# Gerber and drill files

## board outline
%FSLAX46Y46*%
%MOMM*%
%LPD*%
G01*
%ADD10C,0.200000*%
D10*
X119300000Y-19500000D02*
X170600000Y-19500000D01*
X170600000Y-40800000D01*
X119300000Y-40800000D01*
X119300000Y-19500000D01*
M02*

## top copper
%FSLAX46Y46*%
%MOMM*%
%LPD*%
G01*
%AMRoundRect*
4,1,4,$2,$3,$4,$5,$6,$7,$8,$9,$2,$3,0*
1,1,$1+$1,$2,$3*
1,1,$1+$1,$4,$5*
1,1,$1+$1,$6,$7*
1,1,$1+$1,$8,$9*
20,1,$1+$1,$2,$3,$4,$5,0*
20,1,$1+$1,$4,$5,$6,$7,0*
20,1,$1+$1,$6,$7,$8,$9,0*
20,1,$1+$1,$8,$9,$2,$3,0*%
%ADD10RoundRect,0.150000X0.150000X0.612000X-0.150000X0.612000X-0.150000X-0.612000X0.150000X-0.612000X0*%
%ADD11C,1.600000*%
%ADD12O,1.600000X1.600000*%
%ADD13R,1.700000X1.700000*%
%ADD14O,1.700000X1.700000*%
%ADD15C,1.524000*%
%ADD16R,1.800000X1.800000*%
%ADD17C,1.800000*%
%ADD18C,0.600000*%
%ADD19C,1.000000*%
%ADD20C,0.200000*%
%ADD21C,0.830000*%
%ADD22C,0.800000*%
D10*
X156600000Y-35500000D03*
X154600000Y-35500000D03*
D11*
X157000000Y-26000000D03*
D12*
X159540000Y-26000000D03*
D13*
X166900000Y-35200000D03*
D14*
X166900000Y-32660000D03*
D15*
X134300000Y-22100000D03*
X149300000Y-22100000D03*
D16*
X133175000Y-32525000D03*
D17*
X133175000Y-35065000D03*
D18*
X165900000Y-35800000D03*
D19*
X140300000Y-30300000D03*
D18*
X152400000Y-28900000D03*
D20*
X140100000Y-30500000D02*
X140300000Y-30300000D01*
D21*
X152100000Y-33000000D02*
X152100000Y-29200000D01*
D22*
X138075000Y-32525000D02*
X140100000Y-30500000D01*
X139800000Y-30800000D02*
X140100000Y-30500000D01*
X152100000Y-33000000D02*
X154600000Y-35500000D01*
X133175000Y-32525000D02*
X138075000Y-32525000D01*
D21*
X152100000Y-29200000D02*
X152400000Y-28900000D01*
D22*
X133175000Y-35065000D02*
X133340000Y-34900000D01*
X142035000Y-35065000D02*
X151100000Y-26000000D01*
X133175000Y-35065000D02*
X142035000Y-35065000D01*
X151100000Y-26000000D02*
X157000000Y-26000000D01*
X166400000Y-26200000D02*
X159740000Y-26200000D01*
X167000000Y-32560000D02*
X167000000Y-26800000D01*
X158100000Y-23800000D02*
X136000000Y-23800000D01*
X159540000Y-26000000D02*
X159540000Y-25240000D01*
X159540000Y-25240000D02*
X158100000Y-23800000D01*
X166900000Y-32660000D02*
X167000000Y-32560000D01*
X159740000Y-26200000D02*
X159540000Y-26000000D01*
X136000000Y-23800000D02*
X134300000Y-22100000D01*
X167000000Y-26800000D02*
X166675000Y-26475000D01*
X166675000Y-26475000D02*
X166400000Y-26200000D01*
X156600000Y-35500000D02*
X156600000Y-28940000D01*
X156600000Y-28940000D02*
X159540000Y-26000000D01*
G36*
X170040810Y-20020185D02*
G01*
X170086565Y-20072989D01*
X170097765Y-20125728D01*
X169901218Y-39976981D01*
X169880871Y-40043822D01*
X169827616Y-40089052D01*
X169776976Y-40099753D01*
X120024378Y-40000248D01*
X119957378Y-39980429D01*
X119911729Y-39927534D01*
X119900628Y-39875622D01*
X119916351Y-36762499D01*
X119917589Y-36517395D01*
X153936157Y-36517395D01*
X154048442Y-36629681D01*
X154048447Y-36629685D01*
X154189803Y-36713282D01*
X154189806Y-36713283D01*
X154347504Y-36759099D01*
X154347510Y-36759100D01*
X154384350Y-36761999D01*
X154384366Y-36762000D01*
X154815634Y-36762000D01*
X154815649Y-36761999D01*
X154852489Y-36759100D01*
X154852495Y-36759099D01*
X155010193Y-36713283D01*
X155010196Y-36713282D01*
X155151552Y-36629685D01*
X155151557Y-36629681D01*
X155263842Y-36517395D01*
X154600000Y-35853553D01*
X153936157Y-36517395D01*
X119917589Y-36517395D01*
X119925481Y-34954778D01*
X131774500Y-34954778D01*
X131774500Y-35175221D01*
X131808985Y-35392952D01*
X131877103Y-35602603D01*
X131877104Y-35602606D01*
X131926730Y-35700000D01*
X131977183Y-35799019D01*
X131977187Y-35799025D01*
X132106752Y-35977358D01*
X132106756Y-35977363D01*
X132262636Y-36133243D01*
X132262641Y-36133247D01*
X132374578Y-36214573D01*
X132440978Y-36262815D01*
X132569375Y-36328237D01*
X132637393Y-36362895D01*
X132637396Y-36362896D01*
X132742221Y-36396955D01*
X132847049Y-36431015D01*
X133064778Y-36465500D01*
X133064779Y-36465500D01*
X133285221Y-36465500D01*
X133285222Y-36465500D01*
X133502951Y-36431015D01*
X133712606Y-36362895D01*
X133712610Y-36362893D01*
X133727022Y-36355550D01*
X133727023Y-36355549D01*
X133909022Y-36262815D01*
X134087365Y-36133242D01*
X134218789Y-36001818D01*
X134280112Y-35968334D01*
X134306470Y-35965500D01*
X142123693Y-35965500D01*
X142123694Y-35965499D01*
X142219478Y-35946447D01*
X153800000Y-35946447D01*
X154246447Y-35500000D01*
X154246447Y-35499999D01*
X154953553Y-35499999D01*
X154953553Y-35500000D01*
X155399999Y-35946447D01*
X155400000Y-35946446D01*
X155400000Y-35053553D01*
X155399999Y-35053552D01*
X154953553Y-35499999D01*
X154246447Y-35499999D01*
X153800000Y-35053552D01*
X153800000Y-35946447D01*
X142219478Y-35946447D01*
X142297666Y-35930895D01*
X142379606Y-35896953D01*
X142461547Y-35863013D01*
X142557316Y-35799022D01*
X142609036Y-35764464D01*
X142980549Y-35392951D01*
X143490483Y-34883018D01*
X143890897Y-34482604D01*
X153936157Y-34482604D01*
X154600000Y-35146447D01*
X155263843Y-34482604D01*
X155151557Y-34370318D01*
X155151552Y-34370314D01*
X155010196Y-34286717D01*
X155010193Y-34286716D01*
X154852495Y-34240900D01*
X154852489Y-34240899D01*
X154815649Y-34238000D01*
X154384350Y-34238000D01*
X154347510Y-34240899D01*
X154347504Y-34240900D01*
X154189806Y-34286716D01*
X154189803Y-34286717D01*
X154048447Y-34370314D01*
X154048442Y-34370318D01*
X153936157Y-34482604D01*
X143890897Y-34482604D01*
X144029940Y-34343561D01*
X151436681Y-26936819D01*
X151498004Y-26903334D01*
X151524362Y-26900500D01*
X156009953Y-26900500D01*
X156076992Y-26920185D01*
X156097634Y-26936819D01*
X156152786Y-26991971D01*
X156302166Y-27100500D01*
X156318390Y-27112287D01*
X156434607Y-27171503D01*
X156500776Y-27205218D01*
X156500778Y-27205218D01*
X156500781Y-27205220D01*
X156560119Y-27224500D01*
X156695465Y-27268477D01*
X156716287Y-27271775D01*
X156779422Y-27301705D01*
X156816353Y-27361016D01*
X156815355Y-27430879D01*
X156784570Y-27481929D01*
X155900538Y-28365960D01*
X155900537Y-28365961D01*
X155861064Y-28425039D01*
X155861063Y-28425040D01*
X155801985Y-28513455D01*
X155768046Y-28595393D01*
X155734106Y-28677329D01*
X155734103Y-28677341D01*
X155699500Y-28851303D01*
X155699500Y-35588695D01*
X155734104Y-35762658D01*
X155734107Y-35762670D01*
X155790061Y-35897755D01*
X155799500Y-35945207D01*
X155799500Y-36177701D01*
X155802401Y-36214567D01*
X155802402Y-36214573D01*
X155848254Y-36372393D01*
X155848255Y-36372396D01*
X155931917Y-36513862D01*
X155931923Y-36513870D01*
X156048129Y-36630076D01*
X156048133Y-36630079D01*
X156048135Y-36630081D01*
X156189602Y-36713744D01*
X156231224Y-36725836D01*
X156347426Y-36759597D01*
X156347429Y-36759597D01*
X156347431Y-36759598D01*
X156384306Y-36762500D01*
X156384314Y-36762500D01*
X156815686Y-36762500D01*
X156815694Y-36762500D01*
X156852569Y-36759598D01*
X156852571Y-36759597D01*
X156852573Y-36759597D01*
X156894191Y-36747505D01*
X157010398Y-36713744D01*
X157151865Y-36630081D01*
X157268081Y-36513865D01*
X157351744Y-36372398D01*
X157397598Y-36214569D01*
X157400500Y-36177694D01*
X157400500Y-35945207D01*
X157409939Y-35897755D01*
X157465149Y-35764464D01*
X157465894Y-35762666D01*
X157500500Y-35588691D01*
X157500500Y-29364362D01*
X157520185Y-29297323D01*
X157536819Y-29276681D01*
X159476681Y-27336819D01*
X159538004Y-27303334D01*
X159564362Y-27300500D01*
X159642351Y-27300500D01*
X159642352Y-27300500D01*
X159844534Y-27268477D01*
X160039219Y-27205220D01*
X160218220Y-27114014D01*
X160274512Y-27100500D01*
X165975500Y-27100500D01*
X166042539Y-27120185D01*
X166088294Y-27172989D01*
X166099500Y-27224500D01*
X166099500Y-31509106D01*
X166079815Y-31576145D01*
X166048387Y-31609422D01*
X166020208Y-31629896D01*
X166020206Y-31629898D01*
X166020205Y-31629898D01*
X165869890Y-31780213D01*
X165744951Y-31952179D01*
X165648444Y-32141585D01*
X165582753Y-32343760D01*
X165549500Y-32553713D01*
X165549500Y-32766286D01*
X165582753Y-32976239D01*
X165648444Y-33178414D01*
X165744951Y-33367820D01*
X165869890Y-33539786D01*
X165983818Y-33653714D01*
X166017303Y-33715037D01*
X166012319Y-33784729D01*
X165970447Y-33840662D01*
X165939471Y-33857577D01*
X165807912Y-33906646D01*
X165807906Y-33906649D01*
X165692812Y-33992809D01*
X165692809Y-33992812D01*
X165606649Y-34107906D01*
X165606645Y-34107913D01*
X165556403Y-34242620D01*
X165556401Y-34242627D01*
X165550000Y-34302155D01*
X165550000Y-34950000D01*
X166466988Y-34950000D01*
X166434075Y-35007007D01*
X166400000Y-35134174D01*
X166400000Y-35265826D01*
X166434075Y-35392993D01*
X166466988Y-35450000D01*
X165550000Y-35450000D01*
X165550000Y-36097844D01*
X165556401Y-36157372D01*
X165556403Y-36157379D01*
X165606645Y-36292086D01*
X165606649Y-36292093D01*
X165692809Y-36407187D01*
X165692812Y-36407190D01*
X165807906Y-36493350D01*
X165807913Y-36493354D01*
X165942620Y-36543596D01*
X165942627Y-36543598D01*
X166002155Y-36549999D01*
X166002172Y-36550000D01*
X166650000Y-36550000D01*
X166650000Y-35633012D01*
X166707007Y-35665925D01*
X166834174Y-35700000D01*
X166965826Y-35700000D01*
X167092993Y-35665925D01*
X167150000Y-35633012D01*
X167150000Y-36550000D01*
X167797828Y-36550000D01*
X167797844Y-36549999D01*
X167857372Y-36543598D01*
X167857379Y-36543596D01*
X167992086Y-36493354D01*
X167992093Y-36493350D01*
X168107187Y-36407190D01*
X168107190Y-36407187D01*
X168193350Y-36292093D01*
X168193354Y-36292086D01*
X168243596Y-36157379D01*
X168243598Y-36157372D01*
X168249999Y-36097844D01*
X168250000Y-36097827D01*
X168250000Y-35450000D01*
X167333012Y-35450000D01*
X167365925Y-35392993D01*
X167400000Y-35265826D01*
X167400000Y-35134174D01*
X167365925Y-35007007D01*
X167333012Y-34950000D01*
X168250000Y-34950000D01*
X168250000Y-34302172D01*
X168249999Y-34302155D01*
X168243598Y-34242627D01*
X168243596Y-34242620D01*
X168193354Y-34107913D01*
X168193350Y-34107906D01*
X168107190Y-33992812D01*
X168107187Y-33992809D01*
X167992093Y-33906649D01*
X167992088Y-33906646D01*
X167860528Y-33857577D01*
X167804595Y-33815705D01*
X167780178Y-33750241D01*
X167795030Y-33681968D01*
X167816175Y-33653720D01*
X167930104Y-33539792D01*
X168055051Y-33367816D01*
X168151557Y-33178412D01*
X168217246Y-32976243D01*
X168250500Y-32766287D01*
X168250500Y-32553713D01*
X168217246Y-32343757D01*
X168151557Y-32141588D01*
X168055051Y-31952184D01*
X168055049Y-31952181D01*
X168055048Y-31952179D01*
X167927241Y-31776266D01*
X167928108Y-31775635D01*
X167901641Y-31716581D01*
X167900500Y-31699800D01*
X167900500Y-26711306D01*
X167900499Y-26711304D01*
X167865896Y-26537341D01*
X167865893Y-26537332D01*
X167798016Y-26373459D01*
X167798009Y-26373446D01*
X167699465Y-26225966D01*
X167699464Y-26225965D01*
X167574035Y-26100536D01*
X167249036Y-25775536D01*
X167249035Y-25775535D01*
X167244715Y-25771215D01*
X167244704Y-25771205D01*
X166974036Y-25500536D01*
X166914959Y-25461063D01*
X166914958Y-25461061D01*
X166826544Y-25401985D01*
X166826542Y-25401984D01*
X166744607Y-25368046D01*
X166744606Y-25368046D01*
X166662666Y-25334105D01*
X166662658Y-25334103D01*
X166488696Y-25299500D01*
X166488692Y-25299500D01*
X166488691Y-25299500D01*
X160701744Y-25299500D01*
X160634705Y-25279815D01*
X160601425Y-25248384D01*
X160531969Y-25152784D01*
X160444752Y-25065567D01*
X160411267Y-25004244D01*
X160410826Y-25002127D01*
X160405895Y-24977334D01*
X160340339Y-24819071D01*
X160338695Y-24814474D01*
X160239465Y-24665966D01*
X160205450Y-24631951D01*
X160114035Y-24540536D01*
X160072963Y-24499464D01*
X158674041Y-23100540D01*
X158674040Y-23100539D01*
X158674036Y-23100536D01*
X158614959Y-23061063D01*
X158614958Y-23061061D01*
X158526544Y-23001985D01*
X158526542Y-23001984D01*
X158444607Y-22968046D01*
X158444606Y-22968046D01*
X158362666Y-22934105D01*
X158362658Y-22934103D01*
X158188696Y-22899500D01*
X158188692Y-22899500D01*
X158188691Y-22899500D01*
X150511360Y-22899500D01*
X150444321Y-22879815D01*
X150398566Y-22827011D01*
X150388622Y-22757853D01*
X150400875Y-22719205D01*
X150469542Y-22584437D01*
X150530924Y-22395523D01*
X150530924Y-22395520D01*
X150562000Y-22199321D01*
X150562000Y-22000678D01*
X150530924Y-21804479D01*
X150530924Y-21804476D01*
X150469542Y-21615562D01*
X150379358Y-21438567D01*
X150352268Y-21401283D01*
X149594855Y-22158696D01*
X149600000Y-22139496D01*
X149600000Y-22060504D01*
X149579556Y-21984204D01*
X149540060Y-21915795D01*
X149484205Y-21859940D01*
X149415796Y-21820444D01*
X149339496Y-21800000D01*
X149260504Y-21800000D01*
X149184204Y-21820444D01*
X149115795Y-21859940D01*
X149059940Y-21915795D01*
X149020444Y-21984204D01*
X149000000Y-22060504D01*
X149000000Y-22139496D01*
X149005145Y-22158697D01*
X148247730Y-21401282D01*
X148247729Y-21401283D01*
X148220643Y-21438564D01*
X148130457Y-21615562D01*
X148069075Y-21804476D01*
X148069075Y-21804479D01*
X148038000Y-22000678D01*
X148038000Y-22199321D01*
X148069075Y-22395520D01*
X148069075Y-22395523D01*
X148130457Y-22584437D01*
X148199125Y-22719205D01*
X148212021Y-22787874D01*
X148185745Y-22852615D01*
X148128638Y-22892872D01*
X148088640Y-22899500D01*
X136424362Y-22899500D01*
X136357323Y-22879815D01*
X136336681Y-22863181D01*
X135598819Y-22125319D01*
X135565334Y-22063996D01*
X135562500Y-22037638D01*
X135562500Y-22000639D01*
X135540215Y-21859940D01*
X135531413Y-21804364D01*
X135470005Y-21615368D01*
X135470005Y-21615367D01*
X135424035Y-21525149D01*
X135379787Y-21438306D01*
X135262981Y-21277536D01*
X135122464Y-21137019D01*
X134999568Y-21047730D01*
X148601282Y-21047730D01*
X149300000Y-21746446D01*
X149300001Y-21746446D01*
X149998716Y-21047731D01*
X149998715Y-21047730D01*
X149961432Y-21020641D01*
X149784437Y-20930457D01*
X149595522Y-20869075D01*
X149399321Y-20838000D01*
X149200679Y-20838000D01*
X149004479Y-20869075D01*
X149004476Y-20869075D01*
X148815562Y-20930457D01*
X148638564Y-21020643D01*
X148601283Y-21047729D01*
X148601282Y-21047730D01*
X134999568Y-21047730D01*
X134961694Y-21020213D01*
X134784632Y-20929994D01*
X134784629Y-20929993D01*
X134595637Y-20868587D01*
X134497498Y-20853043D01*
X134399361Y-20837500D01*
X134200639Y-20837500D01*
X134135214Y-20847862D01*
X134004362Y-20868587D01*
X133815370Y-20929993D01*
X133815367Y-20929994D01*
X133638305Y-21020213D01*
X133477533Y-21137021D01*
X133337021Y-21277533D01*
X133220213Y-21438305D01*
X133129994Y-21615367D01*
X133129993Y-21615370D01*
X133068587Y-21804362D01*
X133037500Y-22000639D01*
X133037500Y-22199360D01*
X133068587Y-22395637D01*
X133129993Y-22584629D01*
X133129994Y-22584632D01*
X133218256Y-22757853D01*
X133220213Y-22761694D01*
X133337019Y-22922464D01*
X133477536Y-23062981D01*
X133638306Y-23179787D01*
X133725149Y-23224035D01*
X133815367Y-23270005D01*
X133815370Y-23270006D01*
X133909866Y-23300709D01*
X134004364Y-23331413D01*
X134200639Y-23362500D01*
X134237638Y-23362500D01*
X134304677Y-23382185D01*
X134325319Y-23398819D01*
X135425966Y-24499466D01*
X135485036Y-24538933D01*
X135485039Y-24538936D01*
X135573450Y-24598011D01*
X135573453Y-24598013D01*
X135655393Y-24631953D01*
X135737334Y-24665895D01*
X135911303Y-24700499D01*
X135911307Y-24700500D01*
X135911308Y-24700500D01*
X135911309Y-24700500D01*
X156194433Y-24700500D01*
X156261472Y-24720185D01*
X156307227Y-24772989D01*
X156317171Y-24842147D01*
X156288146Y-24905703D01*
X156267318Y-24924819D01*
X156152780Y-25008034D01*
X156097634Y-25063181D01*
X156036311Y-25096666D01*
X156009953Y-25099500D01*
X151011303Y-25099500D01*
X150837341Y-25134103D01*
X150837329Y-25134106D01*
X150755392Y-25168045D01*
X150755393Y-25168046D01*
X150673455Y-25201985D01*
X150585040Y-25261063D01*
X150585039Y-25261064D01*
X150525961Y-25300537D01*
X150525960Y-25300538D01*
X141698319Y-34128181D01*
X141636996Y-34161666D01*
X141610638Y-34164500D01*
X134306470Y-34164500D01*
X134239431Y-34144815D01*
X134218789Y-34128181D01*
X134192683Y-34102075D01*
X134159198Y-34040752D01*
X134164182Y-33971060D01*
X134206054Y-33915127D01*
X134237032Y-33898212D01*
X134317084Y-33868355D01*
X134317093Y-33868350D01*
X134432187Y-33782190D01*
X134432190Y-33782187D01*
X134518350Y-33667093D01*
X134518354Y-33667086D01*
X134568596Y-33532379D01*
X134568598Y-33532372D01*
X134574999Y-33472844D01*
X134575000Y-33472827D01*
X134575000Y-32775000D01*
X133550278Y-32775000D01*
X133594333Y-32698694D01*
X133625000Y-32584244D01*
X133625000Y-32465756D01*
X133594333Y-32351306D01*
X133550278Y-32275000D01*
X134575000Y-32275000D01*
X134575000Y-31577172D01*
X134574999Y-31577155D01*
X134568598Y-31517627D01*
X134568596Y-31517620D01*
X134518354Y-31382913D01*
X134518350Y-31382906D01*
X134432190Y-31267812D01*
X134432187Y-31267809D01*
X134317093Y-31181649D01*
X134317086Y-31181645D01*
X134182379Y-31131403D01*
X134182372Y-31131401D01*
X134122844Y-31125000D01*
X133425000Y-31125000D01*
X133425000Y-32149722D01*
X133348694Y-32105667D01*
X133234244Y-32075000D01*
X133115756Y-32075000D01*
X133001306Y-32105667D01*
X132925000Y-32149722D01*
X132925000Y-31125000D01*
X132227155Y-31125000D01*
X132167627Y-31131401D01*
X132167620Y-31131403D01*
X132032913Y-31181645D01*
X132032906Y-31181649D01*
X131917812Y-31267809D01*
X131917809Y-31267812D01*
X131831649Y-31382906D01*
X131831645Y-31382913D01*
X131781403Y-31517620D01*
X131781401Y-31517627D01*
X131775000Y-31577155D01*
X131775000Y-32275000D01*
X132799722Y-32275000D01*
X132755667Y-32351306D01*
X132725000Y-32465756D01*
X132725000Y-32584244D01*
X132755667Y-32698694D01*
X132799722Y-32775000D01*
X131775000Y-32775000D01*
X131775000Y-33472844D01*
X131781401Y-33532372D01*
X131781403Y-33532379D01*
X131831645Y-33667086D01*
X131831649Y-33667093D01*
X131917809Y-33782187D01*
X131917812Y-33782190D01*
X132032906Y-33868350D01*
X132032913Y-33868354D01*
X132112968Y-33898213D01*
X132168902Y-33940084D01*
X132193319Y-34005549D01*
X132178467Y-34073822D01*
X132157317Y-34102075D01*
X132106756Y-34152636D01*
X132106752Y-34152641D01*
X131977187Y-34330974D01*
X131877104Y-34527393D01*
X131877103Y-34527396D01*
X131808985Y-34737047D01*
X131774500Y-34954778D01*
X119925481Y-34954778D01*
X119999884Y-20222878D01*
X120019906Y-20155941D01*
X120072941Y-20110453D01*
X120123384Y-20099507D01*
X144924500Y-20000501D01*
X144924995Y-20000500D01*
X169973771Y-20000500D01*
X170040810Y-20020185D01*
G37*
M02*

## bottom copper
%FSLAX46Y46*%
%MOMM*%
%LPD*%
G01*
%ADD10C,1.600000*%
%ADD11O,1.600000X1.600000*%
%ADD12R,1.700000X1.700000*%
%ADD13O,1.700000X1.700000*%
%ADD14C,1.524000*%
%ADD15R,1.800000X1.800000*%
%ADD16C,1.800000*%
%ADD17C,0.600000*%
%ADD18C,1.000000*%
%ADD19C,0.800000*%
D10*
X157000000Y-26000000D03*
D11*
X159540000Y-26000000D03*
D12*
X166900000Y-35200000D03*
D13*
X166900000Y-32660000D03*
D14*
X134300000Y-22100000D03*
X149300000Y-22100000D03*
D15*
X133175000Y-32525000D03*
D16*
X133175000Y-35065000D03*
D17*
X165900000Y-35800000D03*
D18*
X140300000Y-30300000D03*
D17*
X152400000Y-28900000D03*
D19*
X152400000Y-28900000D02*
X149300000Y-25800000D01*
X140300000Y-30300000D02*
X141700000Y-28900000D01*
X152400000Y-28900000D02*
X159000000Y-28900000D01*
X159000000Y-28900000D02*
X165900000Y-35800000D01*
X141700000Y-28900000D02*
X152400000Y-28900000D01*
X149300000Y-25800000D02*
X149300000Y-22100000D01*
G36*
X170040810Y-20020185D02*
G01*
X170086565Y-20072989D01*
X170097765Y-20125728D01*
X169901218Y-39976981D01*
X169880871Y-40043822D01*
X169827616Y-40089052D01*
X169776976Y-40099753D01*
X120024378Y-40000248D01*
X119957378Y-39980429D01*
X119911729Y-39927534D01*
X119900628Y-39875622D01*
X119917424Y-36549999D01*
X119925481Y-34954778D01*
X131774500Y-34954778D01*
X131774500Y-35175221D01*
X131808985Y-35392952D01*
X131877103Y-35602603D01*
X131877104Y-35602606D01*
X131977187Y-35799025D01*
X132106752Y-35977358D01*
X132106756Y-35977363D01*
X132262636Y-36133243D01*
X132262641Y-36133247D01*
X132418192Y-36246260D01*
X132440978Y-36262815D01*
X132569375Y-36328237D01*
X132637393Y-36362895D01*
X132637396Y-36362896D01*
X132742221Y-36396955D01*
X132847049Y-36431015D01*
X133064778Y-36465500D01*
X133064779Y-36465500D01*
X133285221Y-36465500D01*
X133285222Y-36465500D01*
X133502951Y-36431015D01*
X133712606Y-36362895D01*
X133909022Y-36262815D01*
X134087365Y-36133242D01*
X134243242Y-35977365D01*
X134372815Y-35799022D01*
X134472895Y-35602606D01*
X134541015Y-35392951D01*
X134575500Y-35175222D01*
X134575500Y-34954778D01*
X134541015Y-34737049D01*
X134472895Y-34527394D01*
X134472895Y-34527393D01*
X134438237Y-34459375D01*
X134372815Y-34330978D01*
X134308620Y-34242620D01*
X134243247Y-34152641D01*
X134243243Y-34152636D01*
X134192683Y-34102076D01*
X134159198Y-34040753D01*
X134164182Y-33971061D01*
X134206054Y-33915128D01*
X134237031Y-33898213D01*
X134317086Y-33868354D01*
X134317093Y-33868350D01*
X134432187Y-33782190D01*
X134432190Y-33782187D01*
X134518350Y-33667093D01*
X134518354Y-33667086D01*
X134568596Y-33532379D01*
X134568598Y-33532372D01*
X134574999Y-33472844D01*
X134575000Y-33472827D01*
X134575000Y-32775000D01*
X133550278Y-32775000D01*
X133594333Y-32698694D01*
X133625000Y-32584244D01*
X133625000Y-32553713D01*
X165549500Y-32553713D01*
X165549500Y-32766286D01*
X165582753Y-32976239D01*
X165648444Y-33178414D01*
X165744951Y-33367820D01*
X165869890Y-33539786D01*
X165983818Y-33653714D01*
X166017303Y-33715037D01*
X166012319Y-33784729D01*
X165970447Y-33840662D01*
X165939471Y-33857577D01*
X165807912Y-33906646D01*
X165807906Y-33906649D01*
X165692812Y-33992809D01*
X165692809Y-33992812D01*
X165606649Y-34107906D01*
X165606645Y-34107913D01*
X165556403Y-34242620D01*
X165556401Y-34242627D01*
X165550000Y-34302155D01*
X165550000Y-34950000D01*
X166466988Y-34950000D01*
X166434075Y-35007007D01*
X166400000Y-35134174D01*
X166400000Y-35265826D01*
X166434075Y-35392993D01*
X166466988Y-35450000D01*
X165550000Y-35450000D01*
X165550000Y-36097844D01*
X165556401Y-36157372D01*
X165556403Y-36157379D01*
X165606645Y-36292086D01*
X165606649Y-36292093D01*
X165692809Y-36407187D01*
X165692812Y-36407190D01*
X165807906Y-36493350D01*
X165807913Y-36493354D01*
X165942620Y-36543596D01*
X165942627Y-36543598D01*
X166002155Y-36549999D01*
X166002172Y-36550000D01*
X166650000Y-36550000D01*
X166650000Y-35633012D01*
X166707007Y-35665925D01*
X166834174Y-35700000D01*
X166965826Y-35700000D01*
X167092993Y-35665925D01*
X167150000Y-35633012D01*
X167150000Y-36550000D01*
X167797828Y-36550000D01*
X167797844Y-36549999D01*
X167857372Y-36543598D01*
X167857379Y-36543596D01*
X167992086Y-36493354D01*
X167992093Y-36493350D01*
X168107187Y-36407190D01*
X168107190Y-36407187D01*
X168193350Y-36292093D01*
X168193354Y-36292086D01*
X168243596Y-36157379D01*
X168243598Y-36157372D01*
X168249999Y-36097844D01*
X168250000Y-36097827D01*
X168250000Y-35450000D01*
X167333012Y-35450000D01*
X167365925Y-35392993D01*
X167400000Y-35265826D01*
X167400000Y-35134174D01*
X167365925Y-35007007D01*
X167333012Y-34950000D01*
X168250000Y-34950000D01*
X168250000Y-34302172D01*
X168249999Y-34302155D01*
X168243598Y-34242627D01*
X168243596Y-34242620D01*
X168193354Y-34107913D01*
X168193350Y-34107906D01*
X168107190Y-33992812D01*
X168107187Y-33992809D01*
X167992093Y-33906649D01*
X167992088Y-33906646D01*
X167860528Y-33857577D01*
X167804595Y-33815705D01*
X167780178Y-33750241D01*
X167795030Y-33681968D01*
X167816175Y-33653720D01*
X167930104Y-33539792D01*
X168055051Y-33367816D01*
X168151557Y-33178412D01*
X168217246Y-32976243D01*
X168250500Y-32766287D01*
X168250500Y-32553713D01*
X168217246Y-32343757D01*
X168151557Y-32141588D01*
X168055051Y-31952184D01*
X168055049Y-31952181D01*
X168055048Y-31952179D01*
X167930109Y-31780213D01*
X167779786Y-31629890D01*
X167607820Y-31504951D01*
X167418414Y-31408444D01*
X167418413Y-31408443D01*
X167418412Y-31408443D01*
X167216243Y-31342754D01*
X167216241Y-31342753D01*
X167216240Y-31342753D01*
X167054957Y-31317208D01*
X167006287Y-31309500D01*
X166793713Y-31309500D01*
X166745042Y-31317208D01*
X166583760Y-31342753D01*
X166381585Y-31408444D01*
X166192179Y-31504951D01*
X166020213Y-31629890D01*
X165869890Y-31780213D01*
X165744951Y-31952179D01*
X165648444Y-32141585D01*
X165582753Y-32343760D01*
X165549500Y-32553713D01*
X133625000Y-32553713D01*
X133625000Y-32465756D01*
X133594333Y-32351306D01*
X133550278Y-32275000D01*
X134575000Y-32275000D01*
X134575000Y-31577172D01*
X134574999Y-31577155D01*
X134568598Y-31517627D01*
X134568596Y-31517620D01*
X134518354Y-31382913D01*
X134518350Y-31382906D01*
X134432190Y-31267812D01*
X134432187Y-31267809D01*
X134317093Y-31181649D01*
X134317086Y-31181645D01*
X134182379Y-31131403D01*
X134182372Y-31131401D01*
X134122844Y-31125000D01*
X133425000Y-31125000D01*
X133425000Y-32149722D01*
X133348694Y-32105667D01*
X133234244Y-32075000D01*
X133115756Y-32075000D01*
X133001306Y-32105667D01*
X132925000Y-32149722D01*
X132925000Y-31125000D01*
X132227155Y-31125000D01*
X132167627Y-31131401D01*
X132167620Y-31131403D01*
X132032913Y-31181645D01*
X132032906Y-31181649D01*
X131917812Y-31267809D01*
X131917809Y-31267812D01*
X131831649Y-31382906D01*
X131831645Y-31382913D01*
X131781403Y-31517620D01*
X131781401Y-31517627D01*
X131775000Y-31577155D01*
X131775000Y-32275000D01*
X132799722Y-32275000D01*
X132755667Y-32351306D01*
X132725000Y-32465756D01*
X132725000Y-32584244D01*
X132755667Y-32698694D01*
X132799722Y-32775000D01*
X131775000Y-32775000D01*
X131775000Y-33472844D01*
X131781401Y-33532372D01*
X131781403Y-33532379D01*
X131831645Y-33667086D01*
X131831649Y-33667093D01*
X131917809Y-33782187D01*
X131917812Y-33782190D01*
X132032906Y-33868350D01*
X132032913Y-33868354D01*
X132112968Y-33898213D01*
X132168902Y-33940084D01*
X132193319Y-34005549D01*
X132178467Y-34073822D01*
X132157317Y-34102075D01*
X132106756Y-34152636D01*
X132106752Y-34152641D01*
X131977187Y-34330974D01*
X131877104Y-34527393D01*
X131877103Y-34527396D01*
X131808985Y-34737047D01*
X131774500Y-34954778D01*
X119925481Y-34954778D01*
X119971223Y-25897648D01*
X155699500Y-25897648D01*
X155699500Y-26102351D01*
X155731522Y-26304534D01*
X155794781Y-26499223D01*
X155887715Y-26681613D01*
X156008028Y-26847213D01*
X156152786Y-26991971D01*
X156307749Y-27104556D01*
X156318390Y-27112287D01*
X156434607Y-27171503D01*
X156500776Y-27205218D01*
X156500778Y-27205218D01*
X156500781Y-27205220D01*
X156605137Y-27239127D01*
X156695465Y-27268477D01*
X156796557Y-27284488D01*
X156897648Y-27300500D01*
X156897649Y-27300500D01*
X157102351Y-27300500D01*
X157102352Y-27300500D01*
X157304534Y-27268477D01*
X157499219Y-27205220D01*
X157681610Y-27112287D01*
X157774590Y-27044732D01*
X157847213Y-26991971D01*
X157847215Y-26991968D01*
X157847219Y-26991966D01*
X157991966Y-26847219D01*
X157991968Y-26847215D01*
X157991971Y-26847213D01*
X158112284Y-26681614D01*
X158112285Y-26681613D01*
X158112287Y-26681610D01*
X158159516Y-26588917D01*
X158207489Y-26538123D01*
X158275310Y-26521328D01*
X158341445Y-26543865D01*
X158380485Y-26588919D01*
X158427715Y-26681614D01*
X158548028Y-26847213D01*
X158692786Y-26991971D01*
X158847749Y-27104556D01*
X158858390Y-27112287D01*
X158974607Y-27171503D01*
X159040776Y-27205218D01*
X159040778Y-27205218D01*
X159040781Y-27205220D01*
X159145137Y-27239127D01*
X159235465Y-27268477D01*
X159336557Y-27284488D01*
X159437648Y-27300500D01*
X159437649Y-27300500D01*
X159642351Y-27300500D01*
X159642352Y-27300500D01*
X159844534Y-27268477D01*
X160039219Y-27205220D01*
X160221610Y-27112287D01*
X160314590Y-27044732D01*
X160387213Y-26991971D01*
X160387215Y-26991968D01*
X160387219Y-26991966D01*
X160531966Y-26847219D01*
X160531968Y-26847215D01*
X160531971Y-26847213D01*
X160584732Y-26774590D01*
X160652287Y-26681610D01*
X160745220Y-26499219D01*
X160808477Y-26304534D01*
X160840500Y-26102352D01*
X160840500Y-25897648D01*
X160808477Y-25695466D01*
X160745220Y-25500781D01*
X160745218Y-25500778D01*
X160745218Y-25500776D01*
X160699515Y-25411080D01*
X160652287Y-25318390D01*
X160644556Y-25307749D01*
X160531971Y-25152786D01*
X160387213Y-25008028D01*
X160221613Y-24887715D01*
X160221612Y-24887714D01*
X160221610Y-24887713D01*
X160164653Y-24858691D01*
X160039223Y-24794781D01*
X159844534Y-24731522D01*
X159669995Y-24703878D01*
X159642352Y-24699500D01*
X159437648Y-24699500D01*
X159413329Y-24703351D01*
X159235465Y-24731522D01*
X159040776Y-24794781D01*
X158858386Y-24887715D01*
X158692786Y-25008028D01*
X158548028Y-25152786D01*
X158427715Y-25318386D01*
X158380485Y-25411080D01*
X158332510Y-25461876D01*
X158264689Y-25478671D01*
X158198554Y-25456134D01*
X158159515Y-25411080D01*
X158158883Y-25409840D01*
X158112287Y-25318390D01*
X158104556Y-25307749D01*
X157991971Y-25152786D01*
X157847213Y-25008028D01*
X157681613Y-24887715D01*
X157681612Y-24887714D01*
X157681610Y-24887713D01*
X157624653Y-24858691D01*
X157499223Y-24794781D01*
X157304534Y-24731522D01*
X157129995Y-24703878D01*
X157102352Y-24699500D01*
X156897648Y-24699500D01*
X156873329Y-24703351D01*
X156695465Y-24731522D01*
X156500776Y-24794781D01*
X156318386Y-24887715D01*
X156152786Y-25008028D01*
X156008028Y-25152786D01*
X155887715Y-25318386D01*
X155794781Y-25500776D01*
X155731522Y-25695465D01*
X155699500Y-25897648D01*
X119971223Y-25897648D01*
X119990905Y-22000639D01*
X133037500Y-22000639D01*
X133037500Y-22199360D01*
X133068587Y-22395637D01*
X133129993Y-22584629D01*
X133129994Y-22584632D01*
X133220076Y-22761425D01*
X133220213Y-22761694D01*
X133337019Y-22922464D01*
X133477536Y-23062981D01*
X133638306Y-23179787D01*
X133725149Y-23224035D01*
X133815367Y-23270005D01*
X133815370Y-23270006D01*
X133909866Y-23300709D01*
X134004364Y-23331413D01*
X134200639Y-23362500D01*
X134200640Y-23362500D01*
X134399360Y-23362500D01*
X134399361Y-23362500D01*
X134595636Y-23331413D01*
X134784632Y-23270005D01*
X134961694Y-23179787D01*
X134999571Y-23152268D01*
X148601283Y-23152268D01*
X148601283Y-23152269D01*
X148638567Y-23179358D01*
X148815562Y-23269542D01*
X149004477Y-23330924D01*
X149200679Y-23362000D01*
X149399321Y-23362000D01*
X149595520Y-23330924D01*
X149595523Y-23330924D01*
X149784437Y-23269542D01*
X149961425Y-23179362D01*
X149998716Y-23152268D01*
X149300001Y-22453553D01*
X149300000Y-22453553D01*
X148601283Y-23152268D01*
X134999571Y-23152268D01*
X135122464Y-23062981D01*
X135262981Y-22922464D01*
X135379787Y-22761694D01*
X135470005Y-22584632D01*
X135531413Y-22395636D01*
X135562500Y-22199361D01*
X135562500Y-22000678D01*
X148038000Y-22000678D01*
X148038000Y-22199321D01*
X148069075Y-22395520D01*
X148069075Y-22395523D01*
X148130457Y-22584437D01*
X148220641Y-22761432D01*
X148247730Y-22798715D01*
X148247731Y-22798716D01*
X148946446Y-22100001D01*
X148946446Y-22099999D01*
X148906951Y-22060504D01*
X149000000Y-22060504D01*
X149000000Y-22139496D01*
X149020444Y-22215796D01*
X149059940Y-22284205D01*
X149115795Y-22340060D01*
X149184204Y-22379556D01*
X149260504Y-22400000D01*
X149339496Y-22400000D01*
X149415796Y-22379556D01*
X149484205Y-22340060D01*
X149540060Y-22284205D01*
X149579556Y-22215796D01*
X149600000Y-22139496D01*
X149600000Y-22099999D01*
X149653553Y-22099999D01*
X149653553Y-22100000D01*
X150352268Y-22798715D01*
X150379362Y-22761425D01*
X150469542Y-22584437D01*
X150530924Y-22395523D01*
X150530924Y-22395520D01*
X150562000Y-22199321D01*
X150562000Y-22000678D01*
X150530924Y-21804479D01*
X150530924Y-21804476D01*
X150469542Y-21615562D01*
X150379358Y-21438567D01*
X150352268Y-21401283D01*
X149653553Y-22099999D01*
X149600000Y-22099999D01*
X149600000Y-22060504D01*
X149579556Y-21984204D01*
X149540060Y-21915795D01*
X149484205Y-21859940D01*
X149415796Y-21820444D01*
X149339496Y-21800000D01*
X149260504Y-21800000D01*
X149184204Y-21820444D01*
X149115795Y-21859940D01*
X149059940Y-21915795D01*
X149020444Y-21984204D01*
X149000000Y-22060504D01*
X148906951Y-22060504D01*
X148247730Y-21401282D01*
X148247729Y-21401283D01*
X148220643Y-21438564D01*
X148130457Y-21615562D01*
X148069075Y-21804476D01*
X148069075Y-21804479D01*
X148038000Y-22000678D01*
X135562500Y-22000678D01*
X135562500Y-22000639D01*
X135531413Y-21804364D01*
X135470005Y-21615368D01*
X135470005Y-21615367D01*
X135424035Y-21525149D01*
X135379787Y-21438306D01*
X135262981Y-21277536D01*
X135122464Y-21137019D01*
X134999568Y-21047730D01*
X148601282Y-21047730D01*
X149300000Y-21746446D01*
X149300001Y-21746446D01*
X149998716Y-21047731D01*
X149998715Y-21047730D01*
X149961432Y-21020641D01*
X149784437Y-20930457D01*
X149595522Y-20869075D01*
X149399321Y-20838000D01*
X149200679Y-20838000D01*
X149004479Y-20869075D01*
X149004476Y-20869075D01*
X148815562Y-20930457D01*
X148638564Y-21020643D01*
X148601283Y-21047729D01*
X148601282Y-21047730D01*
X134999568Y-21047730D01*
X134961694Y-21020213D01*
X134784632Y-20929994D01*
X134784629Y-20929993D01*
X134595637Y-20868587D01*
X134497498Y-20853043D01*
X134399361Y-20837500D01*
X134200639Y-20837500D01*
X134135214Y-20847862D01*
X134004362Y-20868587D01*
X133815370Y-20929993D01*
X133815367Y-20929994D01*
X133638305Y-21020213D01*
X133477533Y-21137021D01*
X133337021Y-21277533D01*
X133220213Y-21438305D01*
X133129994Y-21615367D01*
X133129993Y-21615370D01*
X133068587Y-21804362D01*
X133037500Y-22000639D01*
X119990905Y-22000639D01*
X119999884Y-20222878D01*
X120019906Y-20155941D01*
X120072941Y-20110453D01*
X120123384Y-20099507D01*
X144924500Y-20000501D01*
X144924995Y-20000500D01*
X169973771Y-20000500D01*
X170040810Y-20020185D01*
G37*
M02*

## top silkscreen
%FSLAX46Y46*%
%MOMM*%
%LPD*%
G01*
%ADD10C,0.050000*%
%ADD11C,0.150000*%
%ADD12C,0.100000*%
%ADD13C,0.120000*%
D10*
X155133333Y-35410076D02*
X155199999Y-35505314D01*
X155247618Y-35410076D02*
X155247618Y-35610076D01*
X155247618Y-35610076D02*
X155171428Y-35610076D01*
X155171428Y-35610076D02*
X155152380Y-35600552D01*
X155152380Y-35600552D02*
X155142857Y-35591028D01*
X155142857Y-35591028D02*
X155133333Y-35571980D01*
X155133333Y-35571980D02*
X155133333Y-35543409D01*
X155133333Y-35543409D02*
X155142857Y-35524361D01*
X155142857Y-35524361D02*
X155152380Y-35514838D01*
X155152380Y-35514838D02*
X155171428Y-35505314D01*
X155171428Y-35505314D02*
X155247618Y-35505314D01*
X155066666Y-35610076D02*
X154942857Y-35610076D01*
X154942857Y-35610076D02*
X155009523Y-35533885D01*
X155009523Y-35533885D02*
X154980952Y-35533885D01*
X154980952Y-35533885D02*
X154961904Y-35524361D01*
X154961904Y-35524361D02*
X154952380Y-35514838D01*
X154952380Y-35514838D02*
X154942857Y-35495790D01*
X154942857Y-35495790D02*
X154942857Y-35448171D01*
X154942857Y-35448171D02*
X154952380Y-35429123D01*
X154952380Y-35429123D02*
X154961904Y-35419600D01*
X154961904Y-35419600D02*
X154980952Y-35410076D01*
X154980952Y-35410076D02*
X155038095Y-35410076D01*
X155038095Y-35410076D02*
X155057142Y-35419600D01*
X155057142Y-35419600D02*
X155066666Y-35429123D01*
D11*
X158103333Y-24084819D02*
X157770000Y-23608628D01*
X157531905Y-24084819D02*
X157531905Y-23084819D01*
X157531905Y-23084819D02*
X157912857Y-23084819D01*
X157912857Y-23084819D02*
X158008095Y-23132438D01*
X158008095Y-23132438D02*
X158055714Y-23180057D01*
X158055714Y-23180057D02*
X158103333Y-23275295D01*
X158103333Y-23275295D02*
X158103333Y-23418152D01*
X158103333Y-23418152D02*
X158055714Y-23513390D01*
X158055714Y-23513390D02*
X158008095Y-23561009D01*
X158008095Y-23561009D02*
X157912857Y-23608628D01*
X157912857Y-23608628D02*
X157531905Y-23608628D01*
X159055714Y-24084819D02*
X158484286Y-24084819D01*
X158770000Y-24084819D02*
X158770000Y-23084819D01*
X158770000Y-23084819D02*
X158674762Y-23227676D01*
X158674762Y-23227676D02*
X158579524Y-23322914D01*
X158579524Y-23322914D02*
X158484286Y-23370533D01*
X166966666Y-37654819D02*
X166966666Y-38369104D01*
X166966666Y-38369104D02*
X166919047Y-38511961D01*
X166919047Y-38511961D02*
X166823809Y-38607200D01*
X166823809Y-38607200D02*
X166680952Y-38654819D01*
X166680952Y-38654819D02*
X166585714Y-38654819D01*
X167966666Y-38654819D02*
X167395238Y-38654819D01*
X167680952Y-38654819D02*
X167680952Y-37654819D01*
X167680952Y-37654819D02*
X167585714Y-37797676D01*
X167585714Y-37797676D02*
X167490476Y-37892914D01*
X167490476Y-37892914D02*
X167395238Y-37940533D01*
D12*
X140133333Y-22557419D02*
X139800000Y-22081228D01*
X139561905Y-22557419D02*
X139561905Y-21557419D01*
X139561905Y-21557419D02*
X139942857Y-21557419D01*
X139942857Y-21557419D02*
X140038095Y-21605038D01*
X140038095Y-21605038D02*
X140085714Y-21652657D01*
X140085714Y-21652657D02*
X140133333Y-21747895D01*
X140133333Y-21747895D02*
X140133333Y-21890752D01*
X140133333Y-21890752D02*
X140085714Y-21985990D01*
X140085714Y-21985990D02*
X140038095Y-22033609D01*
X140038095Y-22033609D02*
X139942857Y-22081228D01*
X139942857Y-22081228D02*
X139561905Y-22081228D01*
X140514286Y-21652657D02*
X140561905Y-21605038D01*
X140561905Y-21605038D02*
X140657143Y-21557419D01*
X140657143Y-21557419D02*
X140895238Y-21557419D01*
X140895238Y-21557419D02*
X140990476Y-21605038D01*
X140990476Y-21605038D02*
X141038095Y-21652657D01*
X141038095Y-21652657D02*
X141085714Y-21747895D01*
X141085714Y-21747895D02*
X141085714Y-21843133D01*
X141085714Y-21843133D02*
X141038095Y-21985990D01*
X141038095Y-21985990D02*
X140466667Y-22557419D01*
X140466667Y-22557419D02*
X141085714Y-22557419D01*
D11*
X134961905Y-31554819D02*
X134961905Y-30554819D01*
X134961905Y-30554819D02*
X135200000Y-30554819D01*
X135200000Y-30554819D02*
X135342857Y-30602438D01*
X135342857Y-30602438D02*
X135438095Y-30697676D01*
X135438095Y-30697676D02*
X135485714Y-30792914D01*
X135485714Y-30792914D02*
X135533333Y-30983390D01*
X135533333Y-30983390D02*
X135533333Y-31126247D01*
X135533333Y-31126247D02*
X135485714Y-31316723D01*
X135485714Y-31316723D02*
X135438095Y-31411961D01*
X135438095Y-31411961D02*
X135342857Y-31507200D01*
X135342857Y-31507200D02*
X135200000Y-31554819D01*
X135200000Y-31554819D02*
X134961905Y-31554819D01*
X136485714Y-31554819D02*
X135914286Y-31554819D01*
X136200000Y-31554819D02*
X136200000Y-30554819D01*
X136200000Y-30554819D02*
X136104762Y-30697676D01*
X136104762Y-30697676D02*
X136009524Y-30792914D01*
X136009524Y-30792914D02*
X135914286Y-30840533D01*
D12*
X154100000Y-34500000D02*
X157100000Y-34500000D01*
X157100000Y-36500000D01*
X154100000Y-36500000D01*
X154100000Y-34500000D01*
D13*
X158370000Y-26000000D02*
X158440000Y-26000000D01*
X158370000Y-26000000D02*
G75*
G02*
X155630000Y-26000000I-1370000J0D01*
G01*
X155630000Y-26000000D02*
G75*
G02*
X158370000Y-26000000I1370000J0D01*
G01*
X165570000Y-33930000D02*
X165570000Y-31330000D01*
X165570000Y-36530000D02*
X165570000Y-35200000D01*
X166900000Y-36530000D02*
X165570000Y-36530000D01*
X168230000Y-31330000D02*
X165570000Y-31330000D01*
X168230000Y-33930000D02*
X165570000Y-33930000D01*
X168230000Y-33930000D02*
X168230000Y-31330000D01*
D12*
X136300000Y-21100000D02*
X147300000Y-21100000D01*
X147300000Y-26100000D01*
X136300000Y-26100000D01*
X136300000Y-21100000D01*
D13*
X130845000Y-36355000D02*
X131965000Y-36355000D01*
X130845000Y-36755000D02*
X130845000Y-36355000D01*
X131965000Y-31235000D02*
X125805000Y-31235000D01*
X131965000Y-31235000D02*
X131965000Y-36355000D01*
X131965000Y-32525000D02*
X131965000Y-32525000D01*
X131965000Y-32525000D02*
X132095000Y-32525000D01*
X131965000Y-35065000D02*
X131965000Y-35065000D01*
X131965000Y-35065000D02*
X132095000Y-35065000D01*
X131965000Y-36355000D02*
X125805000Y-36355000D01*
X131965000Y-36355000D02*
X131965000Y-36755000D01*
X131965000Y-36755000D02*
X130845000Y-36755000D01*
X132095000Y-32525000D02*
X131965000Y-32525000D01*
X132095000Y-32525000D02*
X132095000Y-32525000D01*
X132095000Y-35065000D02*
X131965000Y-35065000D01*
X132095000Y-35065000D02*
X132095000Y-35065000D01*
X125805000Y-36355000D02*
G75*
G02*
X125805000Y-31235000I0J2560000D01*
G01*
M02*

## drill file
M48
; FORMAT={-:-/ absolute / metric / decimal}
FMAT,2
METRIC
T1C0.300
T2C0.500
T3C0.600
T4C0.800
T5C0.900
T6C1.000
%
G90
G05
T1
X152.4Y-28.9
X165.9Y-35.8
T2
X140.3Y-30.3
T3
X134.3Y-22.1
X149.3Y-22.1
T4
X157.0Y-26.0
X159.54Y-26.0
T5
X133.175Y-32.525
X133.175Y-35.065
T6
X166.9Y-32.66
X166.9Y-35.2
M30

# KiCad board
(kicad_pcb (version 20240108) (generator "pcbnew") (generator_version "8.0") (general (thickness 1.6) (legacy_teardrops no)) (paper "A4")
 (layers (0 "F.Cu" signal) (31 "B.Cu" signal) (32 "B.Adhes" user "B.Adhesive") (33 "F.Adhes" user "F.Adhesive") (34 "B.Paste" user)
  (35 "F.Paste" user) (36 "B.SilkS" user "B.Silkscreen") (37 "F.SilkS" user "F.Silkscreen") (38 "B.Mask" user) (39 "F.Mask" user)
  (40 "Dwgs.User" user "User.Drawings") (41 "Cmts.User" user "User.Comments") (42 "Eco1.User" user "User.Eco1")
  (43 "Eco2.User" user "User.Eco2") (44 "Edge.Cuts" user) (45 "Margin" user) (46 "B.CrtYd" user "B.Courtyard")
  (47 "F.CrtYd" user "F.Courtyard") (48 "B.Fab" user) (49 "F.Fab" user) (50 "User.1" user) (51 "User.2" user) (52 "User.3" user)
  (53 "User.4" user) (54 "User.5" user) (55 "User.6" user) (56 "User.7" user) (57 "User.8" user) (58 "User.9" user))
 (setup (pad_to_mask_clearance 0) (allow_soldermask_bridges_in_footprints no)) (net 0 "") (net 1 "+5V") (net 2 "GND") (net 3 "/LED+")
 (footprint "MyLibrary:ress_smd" (layer "F.Cu") (at 155.1 35.5 180)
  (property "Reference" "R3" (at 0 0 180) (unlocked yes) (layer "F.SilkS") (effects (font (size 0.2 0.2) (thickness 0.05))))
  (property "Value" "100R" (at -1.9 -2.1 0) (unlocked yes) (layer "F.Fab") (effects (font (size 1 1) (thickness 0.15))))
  (fp_rect (start -2 -1) (end 1 1) (stroke (width 0.1) (type default)) (fill none) (layer "F.SilkS"))
  (pad "1" smd roundrect (at -1.5 0 180) (size 0.6 1.524) (layers "F.Cu" "F.Paste" "F.Mask") (roundrect_rratio 0.25) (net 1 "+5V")
   (thermal_bridge_angle 45))
  (pad "2" smd roundrect (at 0.5 0 180) (size 0.6 1.524) (layers "F.Cu" "F.Paste" "F.Mask") (roundrect_rratio 0.25) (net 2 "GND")
   (thermal_bridge_angle 45)))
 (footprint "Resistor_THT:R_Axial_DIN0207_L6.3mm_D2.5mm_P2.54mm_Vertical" (layer "F.Cu") (at 157 26)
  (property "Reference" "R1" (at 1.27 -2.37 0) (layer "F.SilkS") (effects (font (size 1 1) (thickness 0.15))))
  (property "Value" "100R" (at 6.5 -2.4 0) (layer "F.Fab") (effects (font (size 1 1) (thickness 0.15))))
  (fp_line (start 1.37 0) (end 1.44 0) (stroke (width 0.12) (type solid)) (layer "F.SilkS"))
  (fp_circle (center 0 0) (end 1.37 0) (stroke (width 0.12) (type solid)) (fill none) (layer "F.SilkS"))
  (pad "1" thru_hole circle (at 0 0) (size 1.6 1.6) (drill 0.8) (layers "*.Cu" "*.Mask") (remove_unused_layers no) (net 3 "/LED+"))
  (pad "2" thru_hole oval (at 2.54 0) (size 1.6 1.6) (drill 0.8) (layers "*.Cu" "*.Mask") (remove_unused_layers no) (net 1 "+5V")))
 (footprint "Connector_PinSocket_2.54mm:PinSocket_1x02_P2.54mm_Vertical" (layer "F.Cu") (at 166.9 35.2 180)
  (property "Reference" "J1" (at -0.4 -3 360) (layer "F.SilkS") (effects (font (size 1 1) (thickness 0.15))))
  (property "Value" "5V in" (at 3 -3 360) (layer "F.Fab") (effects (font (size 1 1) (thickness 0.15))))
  (fp_line (start 1.33 1.27) (end 1.33 3.87) (stroke (width 0.12) (type solid)) (layer "F.SilkS"))
  (fp_line (start 1.33 -1.33) (end 1.33 0) (stroke (width 0.12) (type solid)) (layer "F.SilkS"))
  (fp_line (start 0 -1.33) (end 1.33 -1.33) (stroke (width 0.12) (type solid)) (layer "F.SilkS"))
  (fp_line (start -1.33 3.87) (end 1.33 3.87) (stroke (width 0.12) (type solid)) (layer "F.SilkS"))
  (fp_line (start -1.33 1.27) (end 1.33 1.27) (stroke (width 0.12) (type solid)) (layer "F.SilkS"))
  (fp_line (start -1.33 1.27) (end -1.33 3.87) (stroke (width 0.12) (type solid)) (layer "F.SilkS"))
  (pad "1" thru_hole rect (at 0 0 180) (size 1.7 1.7) (drill 1) (layers "*.Cu" "*.Mask") (remove_unused_layers no) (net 2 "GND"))
  (pad "2" thru_hole oval (at 0 2.54 180) (size 1.7 1.7) (drill 1) (layers "*.Cu" "*.Mask") (remove_unused_layers no) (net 1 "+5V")))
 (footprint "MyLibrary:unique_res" (layer "F.Cu") (at 140.3 22.1)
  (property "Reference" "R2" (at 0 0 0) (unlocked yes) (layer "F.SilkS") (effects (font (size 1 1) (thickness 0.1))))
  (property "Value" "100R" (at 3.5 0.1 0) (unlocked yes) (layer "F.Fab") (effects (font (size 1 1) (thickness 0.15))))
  (fp_rect (start -4 -1) (end 7 4) (stroke (width 0.1) (type default)) (fill none) (layer "F.SilkS"))
  (pad "1" thru_hole circle (at -6 0) (size 1.524 1.524) (drill 0.6) (layers "*.Cu" "*.Mask") (remove_unused_layers no) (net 1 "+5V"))
  (pad "2" thru_hole circle (at 9 0) (size 1.524 1.524) (drill 0.6) (layers "*.Cu" "*.Mask") (remove_unused_layers no) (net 2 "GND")))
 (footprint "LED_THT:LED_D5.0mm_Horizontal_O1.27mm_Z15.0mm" (layer "F.Cu") (at 133.175 32.525 -90)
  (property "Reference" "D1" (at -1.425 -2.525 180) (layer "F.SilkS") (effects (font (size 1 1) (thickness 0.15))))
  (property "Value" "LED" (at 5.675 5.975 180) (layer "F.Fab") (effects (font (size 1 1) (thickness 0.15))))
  (fp_line (start 3.83 2.33) (end 3.83 1.21) (stroke (width 0.12) (type solid)) (layer "F.SilkS"))
  (fp_line (start 4.23 2.33) (end 3.83 2.33) (stroke (width 0.12) (type solid)) (layer "F.SilkS"))
  (fp_line (start -1.29 1.21) (end -1.29 7.37) (stroke (width 0.12) (type solid)) (layer "F.SilkS"))
  (fp_line (start -1.29 1.21) (end 3.83 1.21) (stroke (width 0.12) (type solid)) (layer "F.SilkS"))
  (fp_line (start 0 1.21) (end 0 1.21) (stroke (width 0.12) (type solid)) (layer "F.SilkS"))
  (fp_line (start 0 1.21) (end 0 1.08) (stroke (width 0.12) (type solid)) (layer "F.SilkS"))
  (fp_line (start 2.54 1.21) (end 2.54 1.21) (stroke (width 0.12) (type solid)) (layer "F.SilkS"))
  (fp_line (start 2.54 1.21) (end 2.54 1.08) (stroke (width 0.12) (type solid)) (layer "F.SilkS"))
  (fp_line (start 3.83 1.21) (end 3.83 7.37) (stroke (width 0.12) (type solid)) (layer "F.SilkS"))
  (fp_line (start 3.83 1.21) (end 4.23 1.21) (stroke (width 0.12) (type solid)) (layer "F.SilkS"))
  (fp_line (start 4.23 1.21) (end 4.23 2.33) (stroke (width 0.12) (type solid)) (layer "F.SilkS"))
  (fp_line (start 0 1.08) (end 0 1.21) (stroke (width 0.12) (type solid)) (layer "F.SilkS"))
  (fp_line (start 0 1.08) (end 0 1.08) (stroke (width 0.12) (type solid)) (layer "F.SilkS"))
  (fp_line (start 2.54 1.08) (end 2.54 1.21) (stroke (width 0.12) (type solid)) (layer "F.SilkS"))
  (fp_line (start 2.54 1.08) (end 2.54 1.08) (stroke (width 0.12) (type solid)) (layer "F.SilkS"))
  (fp_arc (start 3.83 7.37) (mid 1.27 9.93) (end -1.29 7.37) (stroke (width 0.12) (type solid)) (layer "F.SilkS"))
  (pad "1" thru_hole rect (at 0 0 270) (size 1.8 1.8) (drill 0.9) (layers "*.Cu" "*.Mask") (remove_unused_layers no) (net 2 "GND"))
  (pad "2" thru_hole circle (at 2.54 0 270) (size 1.8 1.8) (drill 0.9) (layers "*.Cu" "*.Mask") (remove_unused_layers no) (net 3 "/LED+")))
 (gr_rect (start 119.3 19.5) (end 170.6 40.8) (stroke (width 0.2) (type default)) (fill none) (layer "Edge.Cuts"))
 (segment (start 140.1 30.5) (end 140.3 30.3) (width 0.2) (layer "F.Cu") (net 2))
 (segment (start 152.1 33) (end 152.1 29.2) (width 0.83) (layer "F.Cu") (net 2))
 (segment (start 138.075 32.525) (end 140.1 30.5) (width 0.8) (layer "F.Cu") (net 2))
 (segment (start 139.8 30.8) (end 140.1 30.5) (width 0.8) (layer "F.Cu") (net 2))
 (segment (start 152.1 33) (end 154.6 35.5) (width 0.8) (layer "F.Cu") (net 2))
 (segment (start 133.175 32.525) (end 138.075 32.525) (width 0.8) (layer "F.Cu") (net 2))
 (segment (start 152.1 29.2) (end 152.4 28.9) (width 0.83) (layer "F.Cu") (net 2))
 (via (at 165.9 35.8) (size 0.6) (drill 0.3) (layers "F.Cu" "B.Cu") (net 2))
 (via (at 140.3 30.3) (size 1) (drill 0.5) (layers "F.Cu" "B.Cu") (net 2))
 (via (at 152.4 28.9) (size 0.6) (drill 0.3) (layers "F.Cu" "B.Cu") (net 2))
 (segment (start 152.4 28.9) (end 149.3 25.8) (width 0.8) (layer "B.Cu") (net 2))
 (segment (start 140.3 30.3) (end 141.7 28.9) (width 0.8) (layer "B.Cu") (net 2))
 (segment (start 152.4 28.9) (end 159 28.9) (width 0.8) (layer "B.Cu") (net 2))
 (segment (start 159 28.9) (end 165.9 35.8) (width 0.8) (layer "B.Cu") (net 2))
 (segment (start 141.7 28.9) (end 152.4 28.9) (width 0.8) (layer "B.Cu") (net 2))
 (segment (start 149.3 25.8) (end 149.3 22.1) (width 0.8) (layer "B.Cu") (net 2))
 (segment (start 133.175 35.065) (end 133.34 34.9) (width 0.8) (layer "F.Cu") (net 3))
 (segment (start 142.035 35.065) (end 151.1 26) (width 0.8) (layer "F.Cu") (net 3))
 (segment (start 133.175 35.065) (end 142.035 35.065) (width 0.8) (layer "F.Cu") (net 3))
 (segment (start 151.1 26) (end 157 26) (width 0.8) (layer "F.Cu") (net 3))
 (segment (start 166.4 26.2) (end 159.74 26.2) (width 0.8) (layer "F.Cu") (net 1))
 (segment (start 167 32.56) (end 167 26.8) (width 0.8) (layer "F.Cu") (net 1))
 (segment (start 158.1 23.8) (end 136 23.8) (width 0.8) (layer "F.Cu") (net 1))
 (segment (start 159.54 26) (end 159.54 25.24) (width 0.8) (layer "F.Cu") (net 1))
 (segment (start 159.54 25.24) (end 158.1 23.8) (width 0.8) (layer "F.Cu") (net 1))
 (segment (start 166.9 32.66) (end 167 32.56) (width 0.8) (layer "F.Cu") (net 1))
 (segment (start 159.74 26.2) (end 159.54 26) (width 0.8) (layer "F.Cu") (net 1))
 (segment (start 136 23.8) (end 134.3 22.1) (width 0.8) (layer "F.Cu") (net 1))
 (segment (start 167 26.8) (end 166.675 26.475) (width 0.8) (layer "F.Cu") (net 1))
 (segment (start 166.675 26.475) (end 166.4 26.2) (width 0.8) (layer "F.Cu") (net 1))
 (segment (start 156.6 35.5) (end 156.6 28.94) (width 0.8) (layer "F.Cu") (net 1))
 (segment (start 156.6 28.94) (end 159.54 26) (width 0.8) (layer "F.Cu") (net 1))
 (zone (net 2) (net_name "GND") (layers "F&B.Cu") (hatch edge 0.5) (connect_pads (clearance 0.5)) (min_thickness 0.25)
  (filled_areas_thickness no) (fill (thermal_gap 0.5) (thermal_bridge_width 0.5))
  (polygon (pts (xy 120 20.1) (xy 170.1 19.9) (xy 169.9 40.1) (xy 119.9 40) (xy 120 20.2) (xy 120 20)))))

